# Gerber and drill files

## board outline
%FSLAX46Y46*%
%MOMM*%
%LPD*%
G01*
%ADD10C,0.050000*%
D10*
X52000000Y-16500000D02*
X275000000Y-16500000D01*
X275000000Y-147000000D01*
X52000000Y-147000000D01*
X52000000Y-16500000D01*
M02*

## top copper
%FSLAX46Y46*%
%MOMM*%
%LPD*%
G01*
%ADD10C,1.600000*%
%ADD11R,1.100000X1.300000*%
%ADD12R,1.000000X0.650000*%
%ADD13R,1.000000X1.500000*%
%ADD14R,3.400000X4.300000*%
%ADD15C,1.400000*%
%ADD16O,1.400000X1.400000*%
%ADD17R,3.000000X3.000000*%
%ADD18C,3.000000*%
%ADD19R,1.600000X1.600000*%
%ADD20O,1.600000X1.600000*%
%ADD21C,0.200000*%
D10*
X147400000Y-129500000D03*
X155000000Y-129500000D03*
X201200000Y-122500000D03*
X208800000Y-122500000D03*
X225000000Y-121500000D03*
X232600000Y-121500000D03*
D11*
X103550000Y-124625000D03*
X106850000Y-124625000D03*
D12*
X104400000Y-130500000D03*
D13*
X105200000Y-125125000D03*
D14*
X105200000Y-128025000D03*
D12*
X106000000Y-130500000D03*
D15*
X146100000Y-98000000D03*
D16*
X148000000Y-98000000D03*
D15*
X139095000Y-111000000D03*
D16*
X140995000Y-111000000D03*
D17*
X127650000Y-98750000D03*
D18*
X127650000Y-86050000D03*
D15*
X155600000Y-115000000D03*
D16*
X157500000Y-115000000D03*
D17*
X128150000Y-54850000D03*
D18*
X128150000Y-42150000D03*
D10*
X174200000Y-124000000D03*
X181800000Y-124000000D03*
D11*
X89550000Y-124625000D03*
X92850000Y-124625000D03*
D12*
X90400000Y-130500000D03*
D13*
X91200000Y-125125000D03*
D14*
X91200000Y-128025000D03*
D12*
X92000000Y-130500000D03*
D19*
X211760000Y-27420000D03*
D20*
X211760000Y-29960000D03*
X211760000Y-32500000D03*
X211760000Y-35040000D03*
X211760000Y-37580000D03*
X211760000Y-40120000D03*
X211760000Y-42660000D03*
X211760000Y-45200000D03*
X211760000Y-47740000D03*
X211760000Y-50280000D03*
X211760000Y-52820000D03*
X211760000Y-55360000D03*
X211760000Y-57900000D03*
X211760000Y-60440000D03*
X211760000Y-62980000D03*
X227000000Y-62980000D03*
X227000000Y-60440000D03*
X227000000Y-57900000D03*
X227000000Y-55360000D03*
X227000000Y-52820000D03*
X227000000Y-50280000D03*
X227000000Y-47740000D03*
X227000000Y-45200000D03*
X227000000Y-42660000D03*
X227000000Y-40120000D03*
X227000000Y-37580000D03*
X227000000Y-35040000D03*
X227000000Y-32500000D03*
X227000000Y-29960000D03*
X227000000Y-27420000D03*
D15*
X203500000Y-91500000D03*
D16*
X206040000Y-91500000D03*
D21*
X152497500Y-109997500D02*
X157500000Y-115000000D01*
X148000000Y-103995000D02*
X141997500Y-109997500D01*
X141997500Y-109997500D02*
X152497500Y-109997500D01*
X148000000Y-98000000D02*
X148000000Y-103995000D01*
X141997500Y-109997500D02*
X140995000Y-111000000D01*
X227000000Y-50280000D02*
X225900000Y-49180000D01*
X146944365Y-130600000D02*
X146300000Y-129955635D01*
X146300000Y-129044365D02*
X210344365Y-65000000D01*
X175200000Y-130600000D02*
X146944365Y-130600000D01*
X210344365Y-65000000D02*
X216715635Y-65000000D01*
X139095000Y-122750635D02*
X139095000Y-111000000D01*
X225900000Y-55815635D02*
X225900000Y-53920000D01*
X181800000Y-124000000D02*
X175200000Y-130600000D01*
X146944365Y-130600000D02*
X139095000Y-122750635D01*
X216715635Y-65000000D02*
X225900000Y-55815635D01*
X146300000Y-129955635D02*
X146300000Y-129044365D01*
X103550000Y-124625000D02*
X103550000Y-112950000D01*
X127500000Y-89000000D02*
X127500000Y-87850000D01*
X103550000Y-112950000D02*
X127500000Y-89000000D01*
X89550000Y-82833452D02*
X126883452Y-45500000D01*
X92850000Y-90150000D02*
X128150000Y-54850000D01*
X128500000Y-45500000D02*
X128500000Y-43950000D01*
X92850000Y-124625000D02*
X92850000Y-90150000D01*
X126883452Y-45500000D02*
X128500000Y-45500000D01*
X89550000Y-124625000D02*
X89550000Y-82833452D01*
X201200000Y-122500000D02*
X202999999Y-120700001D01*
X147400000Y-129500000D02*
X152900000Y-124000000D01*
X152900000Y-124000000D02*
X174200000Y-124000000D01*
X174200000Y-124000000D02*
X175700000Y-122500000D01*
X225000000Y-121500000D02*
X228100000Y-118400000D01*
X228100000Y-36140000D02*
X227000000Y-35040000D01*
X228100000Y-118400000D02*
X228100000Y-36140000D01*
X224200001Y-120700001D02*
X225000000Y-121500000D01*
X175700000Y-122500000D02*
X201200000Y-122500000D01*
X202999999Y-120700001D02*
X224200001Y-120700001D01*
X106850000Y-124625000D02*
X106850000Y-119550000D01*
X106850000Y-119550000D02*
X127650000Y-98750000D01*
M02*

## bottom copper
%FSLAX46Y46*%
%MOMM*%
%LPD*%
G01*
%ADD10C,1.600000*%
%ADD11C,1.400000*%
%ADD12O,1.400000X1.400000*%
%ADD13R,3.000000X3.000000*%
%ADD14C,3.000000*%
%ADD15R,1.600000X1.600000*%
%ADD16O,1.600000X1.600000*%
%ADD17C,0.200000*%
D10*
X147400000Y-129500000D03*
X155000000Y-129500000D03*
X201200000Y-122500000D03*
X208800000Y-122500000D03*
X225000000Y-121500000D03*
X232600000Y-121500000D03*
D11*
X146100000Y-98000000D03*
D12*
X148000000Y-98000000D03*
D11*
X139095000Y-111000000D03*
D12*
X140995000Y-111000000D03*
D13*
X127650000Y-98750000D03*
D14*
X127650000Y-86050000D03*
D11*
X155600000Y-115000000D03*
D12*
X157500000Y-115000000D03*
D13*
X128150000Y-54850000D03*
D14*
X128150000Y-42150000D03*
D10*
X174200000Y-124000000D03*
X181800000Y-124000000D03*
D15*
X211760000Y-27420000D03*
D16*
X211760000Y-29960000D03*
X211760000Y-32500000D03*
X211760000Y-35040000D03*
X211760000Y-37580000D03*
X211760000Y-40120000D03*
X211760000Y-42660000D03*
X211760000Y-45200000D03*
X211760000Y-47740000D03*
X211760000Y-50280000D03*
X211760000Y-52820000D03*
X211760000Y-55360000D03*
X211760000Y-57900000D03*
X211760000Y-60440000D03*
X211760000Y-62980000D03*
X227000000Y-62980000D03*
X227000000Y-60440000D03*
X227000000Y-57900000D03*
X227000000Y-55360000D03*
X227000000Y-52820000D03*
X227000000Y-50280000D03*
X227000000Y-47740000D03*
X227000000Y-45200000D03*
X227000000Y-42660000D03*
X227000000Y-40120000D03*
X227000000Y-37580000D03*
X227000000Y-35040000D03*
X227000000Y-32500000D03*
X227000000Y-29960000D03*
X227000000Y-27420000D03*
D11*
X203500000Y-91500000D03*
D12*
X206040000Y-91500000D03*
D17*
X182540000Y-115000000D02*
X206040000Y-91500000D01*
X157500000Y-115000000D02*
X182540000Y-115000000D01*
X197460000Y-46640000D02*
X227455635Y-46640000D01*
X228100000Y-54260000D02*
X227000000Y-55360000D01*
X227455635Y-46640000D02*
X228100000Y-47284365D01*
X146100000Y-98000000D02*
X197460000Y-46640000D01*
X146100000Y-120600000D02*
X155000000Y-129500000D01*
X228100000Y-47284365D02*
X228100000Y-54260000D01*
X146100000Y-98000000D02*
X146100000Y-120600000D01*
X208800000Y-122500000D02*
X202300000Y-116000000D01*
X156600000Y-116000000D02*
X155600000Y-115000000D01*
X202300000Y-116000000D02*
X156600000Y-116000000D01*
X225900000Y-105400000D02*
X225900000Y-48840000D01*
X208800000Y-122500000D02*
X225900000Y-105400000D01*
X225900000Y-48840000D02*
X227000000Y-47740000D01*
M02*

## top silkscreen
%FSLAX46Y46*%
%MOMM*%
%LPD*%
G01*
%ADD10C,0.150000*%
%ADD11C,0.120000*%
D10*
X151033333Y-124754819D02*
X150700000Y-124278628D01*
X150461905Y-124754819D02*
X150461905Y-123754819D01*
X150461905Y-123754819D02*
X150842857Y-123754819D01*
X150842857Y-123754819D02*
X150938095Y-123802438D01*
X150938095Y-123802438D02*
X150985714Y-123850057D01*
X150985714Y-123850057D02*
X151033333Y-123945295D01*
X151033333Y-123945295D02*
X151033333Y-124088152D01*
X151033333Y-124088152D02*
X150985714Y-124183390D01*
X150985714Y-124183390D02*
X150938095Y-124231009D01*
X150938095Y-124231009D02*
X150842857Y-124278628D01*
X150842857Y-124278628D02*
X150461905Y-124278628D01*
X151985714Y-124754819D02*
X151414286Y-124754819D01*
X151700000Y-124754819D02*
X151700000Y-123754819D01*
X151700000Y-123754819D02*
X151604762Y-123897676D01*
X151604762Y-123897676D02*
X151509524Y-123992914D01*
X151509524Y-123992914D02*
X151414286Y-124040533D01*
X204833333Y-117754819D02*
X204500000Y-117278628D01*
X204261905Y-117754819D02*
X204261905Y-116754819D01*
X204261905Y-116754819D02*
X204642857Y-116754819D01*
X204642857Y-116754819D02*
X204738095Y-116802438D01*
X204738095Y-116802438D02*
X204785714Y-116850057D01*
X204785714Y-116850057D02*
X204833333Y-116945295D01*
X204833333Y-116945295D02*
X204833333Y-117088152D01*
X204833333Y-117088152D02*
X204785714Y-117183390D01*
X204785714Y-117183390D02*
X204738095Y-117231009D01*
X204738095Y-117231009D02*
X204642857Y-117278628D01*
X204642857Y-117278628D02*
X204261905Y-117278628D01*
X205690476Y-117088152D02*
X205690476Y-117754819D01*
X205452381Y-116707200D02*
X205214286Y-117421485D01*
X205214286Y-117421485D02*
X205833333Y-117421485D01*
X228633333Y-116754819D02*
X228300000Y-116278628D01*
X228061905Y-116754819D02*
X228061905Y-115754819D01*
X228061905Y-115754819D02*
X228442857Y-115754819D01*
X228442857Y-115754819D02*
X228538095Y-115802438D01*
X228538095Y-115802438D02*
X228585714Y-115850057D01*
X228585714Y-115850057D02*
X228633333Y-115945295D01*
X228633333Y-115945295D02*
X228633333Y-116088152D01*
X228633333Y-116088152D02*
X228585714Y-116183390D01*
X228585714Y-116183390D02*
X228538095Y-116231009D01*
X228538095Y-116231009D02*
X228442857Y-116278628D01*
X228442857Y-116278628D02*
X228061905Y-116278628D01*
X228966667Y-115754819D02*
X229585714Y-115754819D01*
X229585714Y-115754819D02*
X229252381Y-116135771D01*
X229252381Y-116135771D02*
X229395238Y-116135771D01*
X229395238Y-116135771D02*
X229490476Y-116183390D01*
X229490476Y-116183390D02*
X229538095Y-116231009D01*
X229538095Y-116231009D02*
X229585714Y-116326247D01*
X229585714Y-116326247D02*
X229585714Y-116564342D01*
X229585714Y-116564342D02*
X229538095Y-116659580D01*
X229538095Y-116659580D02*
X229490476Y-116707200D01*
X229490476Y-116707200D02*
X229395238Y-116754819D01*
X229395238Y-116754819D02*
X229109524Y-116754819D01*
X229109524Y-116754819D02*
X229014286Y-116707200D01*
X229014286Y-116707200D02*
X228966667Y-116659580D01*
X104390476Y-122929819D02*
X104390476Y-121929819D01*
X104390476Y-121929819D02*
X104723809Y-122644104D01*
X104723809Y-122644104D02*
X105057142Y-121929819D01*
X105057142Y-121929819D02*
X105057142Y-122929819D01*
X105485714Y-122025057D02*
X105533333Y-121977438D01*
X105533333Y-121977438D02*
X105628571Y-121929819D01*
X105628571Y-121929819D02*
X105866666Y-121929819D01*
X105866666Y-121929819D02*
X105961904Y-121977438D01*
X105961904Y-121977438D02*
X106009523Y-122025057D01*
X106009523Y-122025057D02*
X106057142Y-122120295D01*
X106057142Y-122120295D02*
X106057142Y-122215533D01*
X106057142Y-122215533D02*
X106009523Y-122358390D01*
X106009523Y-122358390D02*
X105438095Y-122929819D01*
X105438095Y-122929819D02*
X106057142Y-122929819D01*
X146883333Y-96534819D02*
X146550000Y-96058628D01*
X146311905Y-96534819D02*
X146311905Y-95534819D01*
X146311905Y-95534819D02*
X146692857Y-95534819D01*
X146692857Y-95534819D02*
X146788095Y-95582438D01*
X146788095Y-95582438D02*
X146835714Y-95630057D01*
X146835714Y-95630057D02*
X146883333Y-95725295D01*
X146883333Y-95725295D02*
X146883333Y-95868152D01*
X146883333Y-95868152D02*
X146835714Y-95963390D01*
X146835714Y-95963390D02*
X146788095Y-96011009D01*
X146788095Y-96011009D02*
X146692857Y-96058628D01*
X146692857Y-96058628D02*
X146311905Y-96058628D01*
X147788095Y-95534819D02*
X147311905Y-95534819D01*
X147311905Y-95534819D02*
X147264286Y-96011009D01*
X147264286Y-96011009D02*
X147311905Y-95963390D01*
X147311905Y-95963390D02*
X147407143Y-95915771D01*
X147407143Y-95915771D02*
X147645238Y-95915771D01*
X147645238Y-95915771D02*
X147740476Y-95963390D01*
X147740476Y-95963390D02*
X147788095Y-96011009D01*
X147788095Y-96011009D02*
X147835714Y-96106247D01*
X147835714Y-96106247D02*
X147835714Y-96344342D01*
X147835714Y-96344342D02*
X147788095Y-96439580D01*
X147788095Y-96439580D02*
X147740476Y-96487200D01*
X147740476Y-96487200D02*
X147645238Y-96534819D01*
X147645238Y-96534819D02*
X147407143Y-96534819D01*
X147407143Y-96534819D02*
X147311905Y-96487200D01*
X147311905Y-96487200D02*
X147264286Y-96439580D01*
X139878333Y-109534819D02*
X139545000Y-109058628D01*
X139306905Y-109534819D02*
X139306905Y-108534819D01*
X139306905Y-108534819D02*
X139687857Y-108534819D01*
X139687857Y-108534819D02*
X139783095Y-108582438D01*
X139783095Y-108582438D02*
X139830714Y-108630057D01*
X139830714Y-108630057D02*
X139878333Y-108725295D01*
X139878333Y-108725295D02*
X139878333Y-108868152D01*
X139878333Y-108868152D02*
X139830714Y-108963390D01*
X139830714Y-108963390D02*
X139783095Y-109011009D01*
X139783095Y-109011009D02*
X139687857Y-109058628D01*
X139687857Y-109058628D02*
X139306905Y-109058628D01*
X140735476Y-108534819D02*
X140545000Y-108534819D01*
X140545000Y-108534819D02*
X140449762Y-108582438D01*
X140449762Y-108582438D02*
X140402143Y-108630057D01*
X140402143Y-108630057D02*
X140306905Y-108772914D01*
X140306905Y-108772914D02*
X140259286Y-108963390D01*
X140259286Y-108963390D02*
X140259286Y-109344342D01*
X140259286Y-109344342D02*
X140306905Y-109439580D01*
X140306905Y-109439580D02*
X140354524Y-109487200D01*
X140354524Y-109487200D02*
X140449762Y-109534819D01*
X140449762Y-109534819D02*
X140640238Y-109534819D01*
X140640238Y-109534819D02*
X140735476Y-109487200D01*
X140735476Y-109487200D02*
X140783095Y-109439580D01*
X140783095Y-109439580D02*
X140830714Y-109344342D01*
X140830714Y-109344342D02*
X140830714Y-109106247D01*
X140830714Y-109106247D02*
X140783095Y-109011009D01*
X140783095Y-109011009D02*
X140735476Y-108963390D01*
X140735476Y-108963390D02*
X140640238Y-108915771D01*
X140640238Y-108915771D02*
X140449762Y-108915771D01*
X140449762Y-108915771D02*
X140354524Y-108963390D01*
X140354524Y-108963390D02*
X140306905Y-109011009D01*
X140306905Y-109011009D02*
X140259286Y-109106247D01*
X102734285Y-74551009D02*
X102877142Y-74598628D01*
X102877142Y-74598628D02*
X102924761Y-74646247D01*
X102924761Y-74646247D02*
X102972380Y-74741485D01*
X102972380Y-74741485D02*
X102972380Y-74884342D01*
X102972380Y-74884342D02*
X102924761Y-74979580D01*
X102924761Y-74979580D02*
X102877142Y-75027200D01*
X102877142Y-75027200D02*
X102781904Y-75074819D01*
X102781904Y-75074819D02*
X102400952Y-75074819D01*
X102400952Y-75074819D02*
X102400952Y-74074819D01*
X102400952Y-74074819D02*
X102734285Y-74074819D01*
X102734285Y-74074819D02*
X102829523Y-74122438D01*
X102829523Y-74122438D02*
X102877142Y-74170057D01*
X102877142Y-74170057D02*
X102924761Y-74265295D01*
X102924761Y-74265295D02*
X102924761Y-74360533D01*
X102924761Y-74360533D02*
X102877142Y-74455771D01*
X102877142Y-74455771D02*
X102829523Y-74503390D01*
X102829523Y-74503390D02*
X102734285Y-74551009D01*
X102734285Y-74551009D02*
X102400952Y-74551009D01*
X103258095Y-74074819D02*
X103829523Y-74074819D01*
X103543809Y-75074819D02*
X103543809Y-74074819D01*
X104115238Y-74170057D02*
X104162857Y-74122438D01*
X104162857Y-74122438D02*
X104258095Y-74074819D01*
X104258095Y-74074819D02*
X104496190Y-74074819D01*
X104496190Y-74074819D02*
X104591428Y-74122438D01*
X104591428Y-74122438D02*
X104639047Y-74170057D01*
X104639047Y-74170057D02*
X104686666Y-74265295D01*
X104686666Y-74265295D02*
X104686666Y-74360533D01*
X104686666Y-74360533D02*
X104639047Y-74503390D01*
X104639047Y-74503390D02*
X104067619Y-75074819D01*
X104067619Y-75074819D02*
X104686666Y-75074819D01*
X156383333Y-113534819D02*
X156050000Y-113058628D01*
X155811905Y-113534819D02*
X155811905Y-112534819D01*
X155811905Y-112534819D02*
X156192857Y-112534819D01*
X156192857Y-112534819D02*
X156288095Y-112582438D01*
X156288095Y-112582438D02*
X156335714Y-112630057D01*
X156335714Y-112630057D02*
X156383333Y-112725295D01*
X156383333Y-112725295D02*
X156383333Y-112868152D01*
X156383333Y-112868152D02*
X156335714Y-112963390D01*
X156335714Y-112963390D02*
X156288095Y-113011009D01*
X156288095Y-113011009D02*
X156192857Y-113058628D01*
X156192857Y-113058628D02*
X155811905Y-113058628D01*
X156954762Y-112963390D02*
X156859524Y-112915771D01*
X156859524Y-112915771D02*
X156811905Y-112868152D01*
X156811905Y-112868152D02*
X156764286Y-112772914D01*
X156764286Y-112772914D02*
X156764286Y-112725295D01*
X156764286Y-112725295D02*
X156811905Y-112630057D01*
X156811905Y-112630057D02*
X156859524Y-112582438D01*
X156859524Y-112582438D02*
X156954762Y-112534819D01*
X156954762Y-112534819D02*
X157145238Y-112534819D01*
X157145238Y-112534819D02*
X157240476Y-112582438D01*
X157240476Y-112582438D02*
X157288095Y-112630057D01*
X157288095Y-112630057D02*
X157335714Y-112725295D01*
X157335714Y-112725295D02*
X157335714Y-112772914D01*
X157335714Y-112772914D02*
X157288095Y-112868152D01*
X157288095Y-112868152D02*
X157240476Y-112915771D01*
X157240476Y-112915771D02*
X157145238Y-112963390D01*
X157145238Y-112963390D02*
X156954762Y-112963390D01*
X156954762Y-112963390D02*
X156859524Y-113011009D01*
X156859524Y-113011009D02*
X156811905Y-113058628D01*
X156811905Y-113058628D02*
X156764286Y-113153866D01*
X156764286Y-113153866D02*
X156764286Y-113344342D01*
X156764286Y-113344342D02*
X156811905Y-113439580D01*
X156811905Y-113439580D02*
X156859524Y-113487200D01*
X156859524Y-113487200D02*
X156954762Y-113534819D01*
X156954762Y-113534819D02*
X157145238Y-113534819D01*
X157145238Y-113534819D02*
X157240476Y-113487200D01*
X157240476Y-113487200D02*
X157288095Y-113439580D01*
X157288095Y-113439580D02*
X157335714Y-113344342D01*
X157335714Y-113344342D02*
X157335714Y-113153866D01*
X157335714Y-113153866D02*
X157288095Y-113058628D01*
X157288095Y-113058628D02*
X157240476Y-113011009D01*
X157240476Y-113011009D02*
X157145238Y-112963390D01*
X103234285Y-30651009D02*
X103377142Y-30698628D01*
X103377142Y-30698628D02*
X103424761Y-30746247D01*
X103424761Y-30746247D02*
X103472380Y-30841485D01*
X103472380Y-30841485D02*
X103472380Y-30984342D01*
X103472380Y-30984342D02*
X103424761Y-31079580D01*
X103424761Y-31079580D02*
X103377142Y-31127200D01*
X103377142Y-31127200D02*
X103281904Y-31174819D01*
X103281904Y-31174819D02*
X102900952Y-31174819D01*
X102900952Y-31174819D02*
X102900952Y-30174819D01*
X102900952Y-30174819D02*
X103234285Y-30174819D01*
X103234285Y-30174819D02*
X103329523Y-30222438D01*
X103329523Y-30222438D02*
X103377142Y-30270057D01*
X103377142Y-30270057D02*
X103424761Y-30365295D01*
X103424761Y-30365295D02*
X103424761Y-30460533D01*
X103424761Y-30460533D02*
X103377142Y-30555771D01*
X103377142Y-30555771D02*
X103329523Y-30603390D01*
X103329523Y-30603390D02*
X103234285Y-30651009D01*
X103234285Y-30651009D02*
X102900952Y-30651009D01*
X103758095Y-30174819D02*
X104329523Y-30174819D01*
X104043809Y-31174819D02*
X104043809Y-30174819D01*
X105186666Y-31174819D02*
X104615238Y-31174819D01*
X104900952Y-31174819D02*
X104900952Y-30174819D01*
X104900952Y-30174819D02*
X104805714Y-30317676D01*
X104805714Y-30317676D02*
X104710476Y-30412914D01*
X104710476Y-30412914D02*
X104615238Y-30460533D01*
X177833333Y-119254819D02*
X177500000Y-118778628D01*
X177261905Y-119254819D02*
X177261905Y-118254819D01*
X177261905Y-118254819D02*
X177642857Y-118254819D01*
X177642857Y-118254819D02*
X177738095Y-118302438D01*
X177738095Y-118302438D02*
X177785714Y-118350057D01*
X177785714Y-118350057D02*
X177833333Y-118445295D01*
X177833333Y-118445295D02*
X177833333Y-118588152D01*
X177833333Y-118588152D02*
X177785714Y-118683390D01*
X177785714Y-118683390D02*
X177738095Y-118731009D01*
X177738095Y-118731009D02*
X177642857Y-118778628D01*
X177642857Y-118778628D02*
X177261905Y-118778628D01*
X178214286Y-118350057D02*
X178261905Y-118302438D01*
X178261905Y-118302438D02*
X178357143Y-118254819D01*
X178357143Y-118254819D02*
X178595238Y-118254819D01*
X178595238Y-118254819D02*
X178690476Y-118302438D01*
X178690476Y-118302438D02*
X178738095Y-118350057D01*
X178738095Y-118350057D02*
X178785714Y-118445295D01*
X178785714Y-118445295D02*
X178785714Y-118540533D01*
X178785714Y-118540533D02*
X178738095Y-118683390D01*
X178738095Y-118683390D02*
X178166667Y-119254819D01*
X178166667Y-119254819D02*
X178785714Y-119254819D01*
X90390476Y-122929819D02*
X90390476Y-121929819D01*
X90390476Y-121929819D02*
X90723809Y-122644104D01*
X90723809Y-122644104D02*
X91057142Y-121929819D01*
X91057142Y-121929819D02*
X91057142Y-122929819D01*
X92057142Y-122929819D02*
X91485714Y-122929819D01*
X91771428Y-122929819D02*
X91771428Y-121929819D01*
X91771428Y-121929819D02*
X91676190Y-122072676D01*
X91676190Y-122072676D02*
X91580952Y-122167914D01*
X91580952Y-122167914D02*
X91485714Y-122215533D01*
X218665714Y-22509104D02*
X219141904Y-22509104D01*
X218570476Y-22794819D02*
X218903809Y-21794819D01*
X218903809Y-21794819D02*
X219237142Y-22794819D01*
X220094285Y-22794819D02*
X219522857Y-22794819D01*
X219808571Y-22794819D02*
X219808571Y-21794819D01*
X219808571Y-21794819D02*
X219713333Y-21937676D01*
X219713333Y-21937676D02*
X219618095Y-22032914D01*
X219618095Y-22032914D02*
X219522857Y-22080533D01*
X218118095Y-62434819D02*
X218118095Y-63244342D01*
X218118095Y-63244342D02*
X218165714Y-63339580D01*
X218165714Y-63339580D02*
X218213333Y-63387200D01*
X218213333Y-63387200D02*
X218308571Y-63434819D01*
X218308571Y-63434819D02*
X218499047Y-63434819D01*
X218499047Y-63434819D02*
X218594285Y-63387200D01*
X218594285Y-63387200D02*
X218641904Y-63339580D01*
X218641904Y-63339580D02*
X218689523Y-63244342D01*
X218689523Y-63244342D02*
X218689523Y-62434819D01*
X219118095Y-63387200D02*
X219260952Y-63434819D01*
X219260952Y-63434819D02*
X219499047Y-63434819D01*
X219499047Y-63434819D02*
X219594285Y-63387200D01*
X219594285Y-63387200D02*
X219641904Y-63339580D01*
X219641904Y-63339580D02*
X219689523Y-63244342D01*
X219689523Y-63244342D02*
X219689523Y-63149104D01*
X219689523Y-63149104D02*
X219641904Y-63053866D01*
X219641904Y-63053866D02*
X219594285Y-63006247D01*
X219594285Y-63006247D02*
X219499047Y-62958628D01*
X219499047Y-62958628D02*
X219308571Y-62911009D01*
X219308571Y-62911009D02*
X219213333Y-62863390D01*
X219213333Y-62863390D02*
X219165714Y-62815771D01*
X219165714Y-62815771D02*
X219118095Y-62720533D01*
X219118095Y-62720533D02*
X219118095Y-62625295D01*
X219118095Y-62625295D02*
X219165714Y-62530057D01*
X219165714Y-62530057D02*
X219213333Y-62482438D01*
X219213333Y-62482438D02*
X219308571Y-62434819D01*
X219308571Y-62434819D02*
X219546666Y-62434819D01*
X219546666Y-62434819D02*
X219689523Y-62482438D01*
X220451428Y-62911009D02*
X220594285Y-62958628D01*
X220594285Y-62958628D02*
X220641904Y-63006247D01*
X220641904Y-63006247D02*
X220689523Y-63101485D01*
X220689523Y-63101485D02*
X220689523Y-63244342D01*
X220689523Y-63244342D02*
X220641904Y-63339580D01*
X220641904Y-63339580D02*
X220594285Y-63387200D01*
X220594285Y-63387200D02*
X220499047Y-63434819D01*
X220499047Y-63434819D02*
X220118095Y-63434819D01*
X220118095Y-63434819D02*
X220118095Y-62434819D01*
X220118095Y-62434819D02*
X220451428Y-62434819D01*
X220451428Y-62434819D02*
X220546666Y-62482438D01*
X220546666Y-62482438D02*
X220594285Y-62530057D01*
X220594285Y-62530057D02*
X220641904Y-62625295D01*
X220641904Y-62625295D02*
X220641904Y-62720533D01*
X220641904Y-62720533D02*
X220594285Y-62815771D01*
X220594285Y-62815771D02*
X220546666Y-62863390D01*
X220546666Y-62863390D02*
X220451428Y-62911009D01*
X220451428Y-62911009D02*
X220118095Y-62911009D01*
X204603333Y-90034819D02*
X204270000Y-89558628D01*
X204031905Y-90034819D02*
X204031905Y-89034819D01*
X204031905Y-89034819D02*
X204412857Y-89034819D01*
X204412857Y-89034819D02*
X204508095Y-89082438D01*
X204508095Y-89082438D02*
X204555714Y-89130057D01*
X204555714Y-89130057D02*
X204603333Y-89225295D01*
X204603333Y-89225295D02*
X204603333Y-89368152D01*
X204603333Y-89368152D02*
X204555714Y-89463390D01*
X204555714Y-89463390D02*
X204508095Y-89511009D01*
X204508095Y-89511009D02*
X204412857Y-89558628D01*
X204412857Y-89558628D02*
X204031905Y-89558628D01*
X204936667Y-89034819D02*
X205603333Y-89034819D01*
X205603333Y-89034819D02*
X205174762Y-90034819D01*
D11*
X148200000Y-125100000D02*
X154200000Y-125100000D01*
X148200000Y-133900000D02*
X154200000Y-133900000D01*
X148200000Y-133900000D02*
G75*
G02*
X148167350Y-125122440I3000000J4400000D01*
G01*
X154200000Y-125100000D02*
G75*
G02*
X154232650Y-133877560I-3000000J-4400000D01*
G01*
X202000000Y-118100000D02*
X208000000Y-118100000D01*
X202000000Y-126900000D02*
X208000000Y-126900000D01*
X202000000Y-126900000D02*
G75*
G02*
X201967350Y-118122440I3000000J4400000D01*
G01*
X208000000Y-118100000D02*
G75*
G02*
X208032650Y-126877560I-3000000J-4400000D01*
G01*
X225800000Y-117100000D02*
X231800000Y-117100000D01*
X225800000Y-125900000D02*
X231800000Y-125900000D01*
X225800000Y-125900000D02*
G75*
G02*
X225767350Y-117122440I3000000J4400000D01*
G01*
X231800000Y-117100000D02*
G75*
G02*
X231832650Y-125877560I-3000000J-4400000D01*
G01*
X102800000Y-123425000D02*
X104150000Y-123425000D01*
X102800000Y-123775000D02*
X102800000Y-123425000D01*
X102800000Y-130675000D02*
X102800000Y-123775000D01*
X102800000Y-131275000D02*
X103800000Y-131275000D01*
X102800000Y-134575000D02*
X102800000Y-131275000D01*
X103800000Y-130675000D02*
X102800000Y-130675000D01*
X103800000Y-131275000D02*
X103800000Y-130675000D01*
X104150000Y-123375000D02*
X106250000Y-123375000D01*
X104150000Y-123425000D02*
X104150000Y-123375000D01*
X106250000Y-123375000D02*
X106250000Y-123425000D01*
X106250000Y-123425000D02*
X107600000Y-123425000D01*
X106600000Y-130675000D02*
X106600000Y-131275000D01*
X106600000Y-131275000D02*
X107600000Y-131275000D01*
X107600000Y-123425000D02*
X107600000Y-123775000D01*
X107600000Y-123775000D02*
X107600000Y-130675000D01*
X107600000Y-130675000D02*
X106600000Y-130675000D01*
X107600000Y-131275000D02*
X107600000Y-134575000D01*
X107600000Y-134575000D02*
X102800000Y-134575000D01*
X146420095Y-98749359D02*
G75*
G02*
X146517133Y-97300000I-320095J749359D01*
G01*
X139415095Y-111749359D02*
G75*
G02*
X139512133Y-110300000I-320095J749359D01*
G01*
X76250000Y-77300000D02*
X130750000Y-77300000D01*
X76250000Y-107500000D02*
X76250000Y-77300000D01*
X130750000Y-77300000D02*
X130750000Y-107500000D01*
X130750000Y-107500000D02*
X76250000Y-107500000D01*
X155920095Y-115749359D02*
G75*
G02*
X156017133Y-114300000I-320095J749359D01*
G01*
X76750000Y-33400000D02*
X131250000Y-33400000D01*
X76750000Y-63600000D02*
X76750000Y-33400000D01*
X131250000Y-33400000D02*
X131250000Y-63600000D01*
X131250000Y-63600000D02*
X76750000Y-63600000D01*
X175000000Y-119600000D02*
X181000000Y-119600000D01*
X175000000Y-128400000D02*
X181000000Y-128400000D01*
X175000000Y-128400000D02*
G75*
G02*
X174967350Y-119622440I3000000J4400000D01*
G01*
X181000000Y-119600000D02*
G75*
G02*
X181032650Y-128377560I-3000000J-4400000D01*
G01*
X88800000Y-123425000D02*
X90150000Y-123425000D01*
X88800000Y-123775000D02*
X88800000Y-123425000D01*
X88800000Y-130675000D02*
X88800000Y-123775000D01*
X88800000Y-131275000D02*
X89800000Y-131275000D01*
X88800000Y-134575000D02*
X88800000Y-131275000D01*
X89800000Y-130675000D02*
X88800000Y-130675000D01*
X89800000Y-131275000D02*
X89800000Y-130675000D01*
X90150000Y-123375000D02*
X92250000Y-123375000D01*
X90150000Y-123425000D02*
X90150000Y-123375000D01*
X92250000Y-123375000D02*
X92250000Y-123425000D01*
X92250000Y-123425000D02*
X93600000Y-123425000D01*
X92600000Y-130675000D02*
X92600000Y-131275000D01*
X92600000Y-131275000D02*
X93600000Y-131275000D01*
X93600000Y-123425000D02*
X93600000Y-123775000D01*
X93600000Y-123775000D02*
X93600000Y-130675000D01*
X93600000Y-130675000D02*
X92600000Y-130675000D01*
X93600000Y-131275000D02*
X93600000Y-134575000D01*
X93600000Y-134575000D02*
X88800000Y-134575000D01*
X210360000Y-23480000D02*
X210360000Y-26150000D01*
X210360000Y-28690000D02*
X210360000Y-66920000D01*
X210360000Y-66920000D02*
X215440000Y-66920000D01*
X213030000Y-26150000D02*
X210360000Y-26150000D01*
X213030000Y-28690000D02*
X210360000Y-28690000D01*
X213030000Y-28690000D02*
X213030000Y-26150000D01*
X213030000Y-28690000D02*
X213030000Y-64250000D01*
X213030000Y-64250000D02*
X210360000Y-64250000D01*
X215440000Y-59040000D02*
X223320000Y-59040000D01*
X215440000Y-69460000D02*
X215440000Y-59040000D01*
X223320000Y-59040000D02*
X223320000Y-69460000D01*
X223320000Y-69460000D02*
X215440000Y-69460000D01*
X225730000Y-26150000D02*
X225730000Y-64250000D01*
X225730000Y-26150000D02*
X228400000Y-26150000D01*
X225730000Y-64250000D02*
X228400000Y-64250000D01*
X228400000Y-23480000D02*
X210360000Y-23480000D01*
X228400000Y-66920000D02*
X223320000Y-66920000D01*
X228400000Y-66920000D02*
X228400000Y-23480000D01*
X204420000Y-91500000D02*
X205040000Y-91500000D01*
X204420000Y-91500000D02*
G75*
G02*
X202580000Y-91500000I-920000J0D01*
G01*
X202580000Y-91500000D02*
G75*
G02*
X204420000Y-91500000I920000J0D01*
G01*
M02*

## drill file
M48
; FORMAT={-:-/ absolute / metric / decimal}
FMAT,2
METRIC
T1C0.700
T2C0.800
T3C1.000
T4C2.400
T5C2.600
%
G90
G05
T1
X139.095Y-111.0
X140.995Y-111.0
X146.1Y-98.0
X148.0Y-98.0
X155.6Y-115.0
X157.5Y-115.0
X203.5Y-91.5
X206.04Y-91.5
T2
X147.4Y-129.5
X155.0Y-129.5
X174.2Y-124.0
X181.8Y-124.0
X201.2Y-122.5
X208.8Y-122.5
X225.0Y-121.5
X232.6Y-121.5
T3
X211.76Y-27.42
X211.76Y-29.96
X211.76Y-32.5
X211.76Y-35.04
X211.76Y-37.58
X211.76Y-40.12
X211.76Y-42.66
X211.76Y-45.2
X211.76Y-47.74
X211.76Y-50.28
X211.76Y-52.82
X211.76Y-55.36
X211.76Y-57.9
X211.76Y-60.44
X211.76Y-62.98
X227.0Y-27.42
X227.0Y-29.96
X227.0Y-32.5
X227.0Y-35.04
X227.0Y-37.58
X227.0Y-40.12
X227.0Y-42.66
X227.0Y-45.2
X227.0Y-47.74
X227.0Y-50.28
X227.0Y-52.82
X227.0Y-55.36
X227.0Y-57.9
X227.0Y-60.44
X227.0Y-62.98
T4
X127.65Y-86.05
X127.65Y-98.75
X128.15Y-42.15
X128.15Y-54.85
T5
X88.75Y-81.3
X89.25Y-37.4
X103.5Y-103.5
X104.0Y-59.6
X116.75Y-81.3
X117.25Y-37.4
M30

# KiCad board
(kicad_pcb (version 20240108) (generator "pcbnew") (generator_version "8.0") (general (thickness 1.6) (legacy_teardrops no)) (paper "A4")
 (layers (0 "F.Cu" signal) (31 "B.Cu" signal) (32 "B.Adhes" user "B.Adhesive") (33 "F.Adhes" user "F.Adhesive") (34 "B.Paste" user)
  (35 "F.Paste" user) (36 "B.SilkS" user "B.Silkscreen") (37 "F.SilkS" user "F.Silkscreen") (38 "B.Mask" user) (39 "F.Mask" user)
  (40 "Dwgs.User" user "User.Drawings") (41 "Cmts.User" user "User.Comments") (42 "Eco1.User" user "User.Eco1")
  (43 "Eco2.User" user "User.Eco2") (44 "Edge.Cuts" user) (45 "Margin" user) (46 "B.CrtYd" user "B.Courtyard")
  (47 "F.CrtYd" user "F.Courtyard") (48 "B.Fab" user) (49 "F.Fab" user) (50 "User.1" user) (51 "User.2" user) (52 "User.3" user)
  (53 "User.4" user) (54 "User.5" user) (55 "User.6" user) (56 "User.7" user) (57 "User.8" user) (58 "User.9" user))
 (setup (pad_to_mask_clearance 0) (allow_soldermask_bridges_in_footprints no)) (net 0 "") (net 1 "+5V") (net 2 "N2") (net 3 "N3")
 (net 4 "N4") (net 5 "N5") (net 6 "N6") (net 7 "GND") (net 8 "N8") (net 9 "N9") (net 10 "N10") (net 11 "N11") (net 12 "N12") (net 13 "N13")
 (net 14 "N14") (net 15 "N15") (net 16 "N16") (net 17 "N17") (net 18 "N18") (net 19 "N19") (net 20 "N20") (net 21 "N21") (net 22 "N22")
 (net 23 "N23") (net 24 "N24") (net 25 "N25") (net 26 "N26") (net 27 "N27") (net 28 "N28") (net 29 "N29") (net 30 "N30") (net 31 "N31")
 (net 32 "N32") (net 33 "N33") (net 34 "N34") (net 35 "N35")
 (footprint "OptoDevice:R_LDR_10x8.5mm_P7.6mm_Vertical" (layer "F.Cu") (at 147.4 129.5)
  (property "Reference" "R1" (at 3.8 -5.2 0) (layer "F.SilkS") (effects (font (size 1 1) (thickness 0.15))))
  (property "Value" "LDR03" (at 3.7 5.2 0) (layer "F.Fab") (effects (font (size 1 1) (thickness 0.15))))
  (fp_line (start 0.8 -4.4) (end 6.8 -4.4) (stroke (width 0.12) (type solid)) (layer "F.SilkS"))
  (fp_line (start 0.8 4.4) (end 6.8 4.4) (stroke (width 0.12) (type solid)) (layer "F.SilkS"))
  (fp_arc (start 0.8 4.4) (mid -1.525374 0.019809) (end 0.76735 -4.37756) (stroke (width 0.12) (type solid)) (layer "F.SilkS"))
  (fp_arc (start 6.8 -4.4) (mid 9.125374 -0.019809) (end 6.83265 4.37756) (stroke (width 0.12) (type solid)) (layer "F.SilkS"))
  (pad "1" thru_hole circle (at 0 0) (size 1.6 1.6) (drill 0.8) (layers "*.Cu" "*.Mask") (remove_unused_layers no) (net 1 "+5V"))
  (pad "2" thru_hole circle (at 7.6 0) (size 1.6 1.6) (drill 0.8) (layers "*.Cu" "*.Mask") (remove_unused_layers no) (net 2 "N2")))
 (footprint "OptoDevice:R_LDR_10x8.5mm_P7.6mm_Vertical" (layer "F.Cu") (at 201.2 122.5)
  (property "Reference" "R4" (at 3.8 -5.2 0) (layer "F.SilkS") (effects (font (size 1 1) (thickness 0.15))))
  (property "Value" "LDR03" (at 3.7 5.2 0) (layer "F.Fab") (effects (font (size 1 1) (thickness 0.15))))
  (fp_line (start 0.8 -4.4) (end 6.8 -4.4) (stroke (width 0.12) (type solid)) (layer "F.SilkS"))
  (fp_line (start 0.8 4.4) (end 6.8 4.4) (stroke (width 0.12) (type solid)) (layer "F.SilkS"))
  (fp_arc (start 0.8 4.4) (mid -1.525374 0.019809) (end 0.76735 -4.37756) (stroke (width 0.12) (type solid)) (layer "F.SilkS"))
  (fp_arc (start 6.8 -4.4) (mid 9.125374 -0.019809) (end 6.83265 4.37756) (stroke (width 0.12) (type solid)) (layer "F.SilkS"))
  (pad "1" thru_hole circle (at 0 0) (size 1.6 1.6) (drill 0.8) (layers "*.Cu" "*.Mask") (remove_unused_layers no) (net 1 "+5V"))
  (pad "2" thru_hole circle (at 7.6 0) (size 1.6 1.6) (drill 0.8) (layers "*.Cu" "*.Mask") (remove_unused_layers no) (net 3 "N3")))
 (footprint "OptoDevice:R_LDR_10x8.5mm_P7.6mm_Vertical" (layer "F.Cu") (at 225 121.5)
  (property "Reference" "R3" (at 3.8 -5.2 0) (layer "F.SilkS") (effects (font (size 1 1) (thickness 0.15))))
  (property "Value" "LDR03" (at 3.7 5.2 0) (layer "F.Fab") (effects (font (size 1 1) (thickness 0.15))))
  (fp_line (start 0.8 -4.4) (end 6.8 -4.4) (stroke (width 0.12) (type solid)) (layer "F.SilkS"))
  (fp_line (start 0.8 4.4) (end 6.8 4.4) (stroke (width 0.12) (type solid)) (layer "F.SilkS"))
  (fp_arc (start 0.8 4.4) (mid -1.525374 0.019809) (end 0.76735 -4.37756) (stroke (width 0.12) (type solid)) (layer "F.SilkS"))
  (fp_arc (start 6.8 -4.4) (mid 9.125374 -0.019809) (end 6.83265 4.37756) (stroke (width 0.12) (type solid)) (layer "F.SilkS"))
  (pad "1" thru_hole circle (at 0 0) (size 1.6 1.6) (drill 0.8) (layers "*.Cu" "*.Mask") (remove_unused_layers no) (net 1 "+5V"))
  (pad "2" thru_hole circle (at 7.6 0) (size 1.6 1.6) (drill 0.8) (layers "*.Cu" "*.Mask") (remove_unused_layers no) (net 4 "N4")))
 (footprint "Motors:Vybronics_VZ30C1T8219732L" (layer "F.Cu") (at 105.2 128.975)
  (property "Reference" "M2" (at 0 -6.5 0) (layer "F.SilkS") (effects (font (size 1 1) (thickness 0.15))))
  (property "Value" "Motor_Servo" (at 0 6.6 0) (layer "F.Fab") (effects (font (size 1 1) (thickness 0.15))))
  (fp_line (start -2.4 -5.55) (end -1.05 -5.55) (stroke (width 0.12) (type solid)) (layer "F.SilkS"))
  (fp_line (start -2.4 -5.2) (end -2.4 -5.55) (stroke (width 0.12) (type solid)) (layer "F.SilkS"))
  (fp_line (start -2.4 1.7) (end -2.4 -5.2) (stroke (width 0.12) (type solid)) (layer "F.SilkS"))
  (fp_line (start -2.4 2.3) (end -1.4 2.3) (stroke (width 0.12) (type solid)) (layer "F.SilkS"))
  (fp_line (start -2.4 5.6) (end -2.4 2.3) (stroke (width 0.12) (type solid)) (layer "F.SilkS"))
  (fp_line (start -1.4 1.7) (end -2.4 1.7) (stroke (width 0.12) (type solid)) (layer "F.SilkS"))
  (fp_line (start -1.4 2.3) (end -1.4 1.7) (stroke (width 0.12) (type solid)) (layer "F.SilkS"))
  (fp_line (start -1.05 -5.6) (end 1.05 -5.6) (stroke (width 0.12) (type solid)) (layer "F.SilkS"))
  (fp_line (start -1.05 -5.55) (end -1.05 -5.6) (stroke (width 0.12) (type solid)) (layer "F.SilkS"))
  (fp_line (start 1.05 -5.6) (end 1.05 -5.55) (stroke (width 0.12) (type solid)) (layer "F.SilkS"))
  (fp_line (start 1.05 -5.55) (end 2.4 -5.55) (stroke (width 0.12) (type solid)) (layer "F.SilkS"))
  (fp_line (start 1.4 1.7) (end 1.4 2.3) (stroke (width 0.12) (type solid)) (layer "F.SilkS"))
  (fp_line (start 1.4 2.3) (end 2.4 2.3) (stroke (width 0.12) (type solid)) (layer "F.SilkS"))
  (fp_line (start 2.4 -5.55) (end 2.4 -5.2) (stroke (width 0.12) (type solid)) (layer "F.SilkS"))
  (fp_line (start 2.4 -5.2) (end 2.4 1.7) (stroke (width 0.12) (type solid)) (layer "F.SilkS"))
  (fp_line (start 2.4 1.7) (end 1.4 1.7) (stroke (width 0.12) (type solid)) (layer "F.SilkS"))
  (fp_line (start 2.4 2.3) (end 2.4 5.6) (stroke (width 0.12) (type solid)) (layer "F.SilkS"))
  (fp_line (start 2.4 5.6) (end -2.4 5.6) (stroke (width 0.12) (type solid)) (layer "F.SilkS"))
  (pad "" smd rect (at -0.85 -2.315 270) (size 1.07 1.4) (layers "F.Paste"))
  (pad "" smd rect (at -0.85 -0.905 270) (size 1.07 1.4) (layers "F.Paste"))
  (pad "" smd rect (at -0.85 0.505 270) (size 1.07 1.4) (layers "F.Paste"))
  (pad "" smd rect (at 0.85 -2.315 270) (size 1.07 1.4) (layers "F.Paste"))
  (pad "" smd rect (at 0.85 -0.905 270) (size 1.07 1.4) (layers "F.Paste"))
  (pad "" smd rect (at 0.85 0.505 270) (size 1.07 1.4) (layers "F.Paste"))
  (pad "1" smd rect (at -1.65 -4.35 270) (size 1.3 1.1) (layers "F.Cu" "F.Paste" "F.Mask") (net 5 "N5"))
  (pad "2" smd rect (at 1.65 -4.35 270) (size 1.3 1.1) (layers "F.Cu" "F.Paste" "F.Mask") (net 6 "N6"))
  (pad "SH" smd rect (at -0.8 1.525) (size 1 0.65) (layers "F.Cu" "F.Paste" "F.Mask"))
  (pad "SH" smd rect (at 0 -3.85 270) (size 1.5 1) (layers "F.Cu" "F.Paste" "F.Mask"))
  (pad "SH" smd rect (at 0 -0.95 270) (size 4.3 3.4) (layers "F.Cu" "F.Mask"))
  (pad "SH" smd rect (at 0.8 1.525) (size 1 0.65) (layers "F.Cu" "F.Paste" "F.Mask")))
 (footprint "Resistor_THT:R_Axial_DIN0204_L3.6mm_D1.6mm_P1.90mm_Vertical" (layer "F.Cu") (at 146.1 98)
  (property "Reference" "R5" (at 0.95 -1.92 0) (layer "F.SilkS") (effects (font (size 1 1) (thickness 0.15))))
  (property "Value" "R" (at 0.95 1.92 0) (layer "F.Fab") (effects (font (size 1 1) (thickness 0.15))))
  (fp_arc (start 0.320095 0.749359) (mid -0.813042 -0.054435) (end 0.417133 -0.7) (stroke (width 0.12) (type solid)) (layer "F.SilkS"))
  (pad "1" thru_hole circle (at 0 0) (size 1.4 1.4) (drill 0.7) (layers "*.Cu" "*.Mask") (remove_unused_layers no) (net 2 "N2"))
  (pad "2" thru_hole oval (at 1.9 0) (size 1.4 1.4) (drill 0.7) (layers "*.Cu" "*.Mask") (remove_unused_layers no) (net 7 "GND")))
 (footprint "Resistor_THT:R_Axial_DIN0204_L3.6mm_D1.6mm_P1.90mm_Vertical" (layer "F.Cu") (at 139.095 111)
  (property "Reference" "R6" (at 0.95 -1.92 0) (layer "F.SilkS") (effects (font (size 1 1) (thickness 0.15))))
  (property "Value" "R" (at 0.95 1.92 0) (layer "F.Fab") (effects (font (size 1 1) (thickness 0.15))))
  (fp_arc (start 0.320095 0.749359) (mid -0.813042 -0.054435) (end 0.417133 -0.7) (stroke (width 0.12) (type solid)) (layer "F.SilkS"))
  (pad "1" thru_hole circle (at 0 0) (size 1.4 1.4) (drill 0.7) (layers "*.Cu" "*.Mask") (remove_unused_layers no) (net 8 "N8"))
  (pad "2" thru_hole oval (at 1.9 0) (size 1.4 1.4) (drill 0.7) (layers "*.Cu" "*.Mask") (remove_unused_layers no) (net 7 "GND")))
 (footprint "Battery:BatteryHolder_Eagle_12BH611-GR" (layer "F.Cu") (at 127.65 98.75)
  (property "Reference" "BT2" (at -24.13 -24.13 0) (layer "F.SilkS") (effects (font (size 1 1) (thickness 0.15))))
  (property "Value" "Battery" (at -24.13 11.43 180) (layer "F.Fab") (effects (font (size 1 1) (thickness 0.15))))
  (fp_line (start -51.4 -21.45) (end 3.1 -21.45) (stroke (width 0.12) (type solid)) (layer "F.SilkS"))
  (fp_line (start -51.4 8.75) (end -51.4 -21.45) (stroke (width 0.12) (type solid)) (layer "F.SilkS"))
  (fp_line (start 3.1 -21.45) (end 3.1 8.75) (stroke (width 0.12) (type solid)) (layer "F.SilkS"))
  (fp_line (start 3.1 8.75) (end -51.4 8.75) (stroke (width 0.12) (type solid)) (layer "F.SilkS"))
  (pad "" np_thru_hole circle (at -38.9 -17.45) (size 2.6 2.6) (drill 2.6) (layers "*.Cu" "*.Mask"))
  (pad "" np_thru_hole circle (at -24.15 4.75) (size 2.6 2.6) (drill 2.6) (layers "*.Cu" "*.Mask"))
  (pad "" np_thru_hole circle (at -10.9 -17.45) (size 2.6 2.6) (drill 2.6) (layers "*.Cu" "*.Mask"))
  (pad "1" thru_hole rect (at 0 0) (size 3 3) (drill 2.4) (layers "*.Cu" "*.Mask") (remove_unused_layers no) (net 6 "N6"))
  (pad "2" thru_hole circle (at 0 -12.7) (size 3 3) (drill 2.4) (layers "*.Cu" "*.Mask") (remove_unused_layers no) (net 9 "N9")))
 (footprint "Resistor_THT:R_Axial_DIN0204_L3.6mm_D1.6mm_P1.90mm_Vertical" (layer "F.Cu") (at 155.6 115)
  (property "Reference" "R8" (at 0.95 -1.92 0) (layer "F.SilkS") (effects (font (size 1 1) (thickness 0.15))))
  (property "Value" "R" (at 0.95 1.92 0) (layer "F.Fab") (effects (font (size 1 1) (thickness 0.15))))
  (fp_arc (start 0.320095 0.749359) (mid -0.813042 -0.054435) (end 0.417133 -0.7) (stroke (width 0.12) (type solid)) (layer "F.SilkS"))
  (pad "1" thru_hole circle (at 0 0) (size 1.4 1.4) (drill 0.7) (layers "*.Cu" "*.Mask") (remove_unused_layers no) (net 3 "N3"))
  (pad "2" thru_hole oval (at 1.9 0) (size 1.4 1.4) (drill 0.7) (layers "*.Cu" "*.Mask") (remove_unused_layers no) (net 7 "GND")))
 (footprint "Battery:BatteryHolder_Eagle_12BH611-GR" (layer "F.Cu") (at 128.15 54.85)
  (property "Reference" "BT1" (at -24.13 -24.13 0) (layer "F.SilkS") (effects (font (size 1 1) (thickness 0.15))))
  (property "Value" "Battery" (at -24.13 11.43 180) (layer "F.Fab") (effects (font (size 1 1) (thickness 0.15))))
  (fp_line (start -51.4 -21.45) (end 3.1 -21.45) (stroke (width 0.12) (type solid)) (layer "F.SilkS"))
  (fp_line (start -51.4 8.75) (end -51.4 -21.45) (stroke (width 0.12) (type solid)) (layer "F.SilkS"))
  (fp_line (start 3.1 -21.45) (end 3.1 8.75) (stroke (width 0.12) (type solid)) (layer "F.SilkS"))
  (fp_line (start 3.1 8.75) (end -51.4 8.75) (stroke (width 0.12) (type solid)) (layer "F.SilkS"))
  (pad "" np_thru_hole circle (at -38.9 -17.45) (size 2.6 2.6) (drill 2.6) (layers "*.Cu" "*.Mask"))
  (pad "" np_thru_hole circle (at -24.15 4.75) (size 2.6 2.6) (drill 2.6) (layers "*.Cu" "*.Mask"))
  (pad "" np_thru_hole circle (at -10.9 -17.45) (size 2.6 2.6) (drill 2.6) (layers "*.Cu" "*.Mask"))
  (pad "1" thru_hole rect (at 0 0) (size 3 3) (drill 2.4) (layers "*.Cu" "*.Mask") (remove_unused_layers no) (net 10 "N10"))
  (pad "2" thru_hole circle (at 0 -12.7) (size 3 3) (drill 2.4) (layers "*.Cu" "*.Mask") (remove_unused_layers no) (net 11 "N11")))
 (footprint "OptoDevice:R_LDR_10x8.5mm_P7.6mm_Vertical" (layer "F.Cu") (at 174.2 124)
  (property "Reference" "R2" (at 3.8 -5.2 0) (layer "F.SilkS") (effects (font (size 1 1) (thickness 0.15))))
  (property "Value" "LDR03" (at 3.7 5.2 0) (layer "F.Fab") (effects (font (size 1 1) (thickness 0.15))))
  (fp_line (start 0.8 -4.4) (end 6.8 -4.4) (stroke (width 0.12) (type solid)) (layer "F.SilkS"))
  (fp_line (start 0.8 4.4) (end 6.8 4.4) (stroke (width 0.12) (type solid)) (layer "F.SilkS"))
  (fp_arc (start 0.8 4.4) (mid -1.525374 0.019809) (end 0.76735 -4.37756) (stroke (width 0.12) (type solid)) (layer "F.SilkS"))
  (fp_arc (start 6.8 -4.4) (mid 9.125374 -0.019809) (end 6.83265 4.37756) (stroke (width 0.12) (type solid)) (layer "F.SilkS"))
  (pad "1" thru_hole circle (at 0 0) (size 1.6 1.6) (drill 0.8) (layers "*.Cu" "*.Mask") (remove_unused_layers no) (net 1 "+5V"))
  (pad "2" thru_hole circle (at 7.6 0) (size 1.6 1.6) (drill 0.8) (layers "*.Cu" "*.Mask") (remove_unused_layers no) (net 8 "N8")))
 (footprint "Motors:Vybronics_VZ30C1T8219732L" (layer "F.Cu") (at 91.2 128.975)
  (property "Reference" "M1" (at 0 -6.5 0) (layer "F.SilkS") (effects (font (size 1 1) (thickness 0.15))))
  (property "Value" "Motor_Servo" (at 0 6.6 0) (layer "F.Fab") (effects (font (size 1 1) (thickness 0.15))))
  (fp_line (start -2.4 -5.55) (end -1.05 -5.55) (stroke (width 0.12) (type solid)) (layer "F.SilkS"))
  (fp_line (start -2.4 -5.2) (end -2.4 -5.55) (stroke (width 0.12) (type solid)) (layer "F.SilkS"))
  (fp_line (start -2.4 1.7) (end -2.4 -5.2) (stroke (width 0.12) (type solid)) (layer "F.SilkS"))
  (fp_line (start -2.4 2.3) (end -1.4 2.3) (stroke (width 0.12) (type solid)) (layer "F.SilkS"))
  (fp_line (start -2.4 5.6) (end -2.4 2.3) (stroke (width 0.12) (type solid)) (layer "F.SilkS"))
  (fp_line (start -1.4 1.7) (end -2.4 1.7) (stroke (width 0.12) (type solid)) (layer "F.SilkS"))
  (fp_line (start -1.4 2.3) (end -1.4 1.7) (stroke (width 0.12) (type solid)) (layer "F.SilkS"))
  (fp_line (start -1.05 -5.6) (end 1.05 -5.6) (stroke (width 0.12) (type solid)) (layer "F.SilkS"))
  (fp_line (start -1.05 -5.55) (end -1.05 -5.6) (stroke (width 0.12) (type solid)) (layer "F.SilkS"))
  (fp_line (start 1.05 -5.6) (end 1.05 -5.55) (stroke (width 0.12) (type solid)) (layer "F.SilkS"))
  (fp_line (start 1.05 -5.55) (end 2.4 -5.55) (stroke (width 0.12) (type solid)) (layer "F.SilkS"))
  (fp_line (start 1.4 1.7) (end 1.4 2.3) (stroke (width 0.12) (type solid)) (layer "F.SilkS"))
  (fp_line (start 1.4 2.3) (end 2.4 2.3) (stroke (width 0.12) (type solid)) (layer "F.SilkS"))
  (fp_line (start 2.4 -5.55) (end 2.4 -5.2) (stroke (width 0.12) (type solid)) (layer "F.SilkS"))
  (fp_line (start 2.4 -5.2) (end 2.4 1.7) (stroke (width 0.12) (type solid)) (layer "F.SilkS"))
  (fp_line (start 2.4 1.7) (end 1.4 1.7) (stroke (width 0.12) (type solid)) (layer "F.SilkS"))
  (fp_line (start 2.4 2.3) (end 2.4 5.6) (stroke (width 0.12) (type solid)) (layer "F.SilkS"))
  (fp_line (start 2.4 5.6) (end -2.4 5.6) (stroke (width 0.12) (type solid)) (layer "F.SilkS"))
  (pad "" smd rect (at -0.85 -2.315 270) (size 1.07 1.4) (layers "F.Paste"))
  (pad "" smd rect (at -0.85 -0.905 270) (size 1.07 1.4) (layers "F.Paste"))
  (pad "" smd rect (at -0.85 0.505 270) (size 1.07 1.4) (layers "F.Paste"))
  (pad "" smd rect (at 0.85 -2.315 270) (size 1.07 1.4) (layers "F.Paste"))
  (pad "" smd rect (at 0.85 -0.905 270) (size 1.07 1.4) (layers "F.Paste"))
  (pad "" smd rect (at 0.85 0.505 270) (size 1.07 1.4) (layers "F.Paste"))
  (pad "1" smd rect (at -1.65 -4.35 270) (size 1.3 1.1) (layers "F.Cu" "F.Paste" "F.Mask") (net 10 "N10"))
  (pad "2" smd rect (at 1.65 -4.35 270) (size 1.3 1.1) (layers "F.Cu" "F.Paste" "F.Mask") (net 10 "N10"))
  (pad "SH" smd rect (at -0.8 1.525) (size 1 0.65) (layers "F.Cu" "F.Paste" "F.Mask"))
  (pad "SH" smd rect (at 0 -3.85 270) (size 1.5 1) (layers "F.Cu" "F.Paste" "F.Mask"))
  (pad "SH" smd rect (at 0 -0.95 270) (size 4.3 3.4) (layers "F.Cu" "F.Mask"))
  (pad "SH" smd rect (at 0.8 1.525) (size 1 0.65) (layers "F.Cu" "F.Paste" "F.Mask")))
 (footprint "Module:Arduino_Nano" (layer "F.Cu") (at 211.76 27.42)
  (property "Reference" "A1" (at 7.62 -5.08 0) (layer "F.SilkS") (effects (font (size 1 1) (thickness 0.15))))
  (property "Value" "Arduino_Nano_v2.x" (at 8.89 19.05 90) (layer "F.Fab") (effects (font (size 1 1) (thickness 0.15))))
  (fp_line (start -1.4 -3.94) (end -1.4 -1.27) (stroke (width 0.12) (type solid)) (layer "F.SilkS"))
  (fp_line (start -1.4 1.27) (end -1.4 39.5) (stroke (width 0.12) (type solid)) (layer "F.SilkS"))
  (fp_line (start -1.4 39.5) (end 3.68 39.5) (stroke (width 0.12) (type solid)) (layer "F.SilkS"))
  (fp_line (start 1.27 -1.27) (end -1.4 -1.27) (stroke (width 0.12) (type solid)) (layer "F.SilkS"))
  (fp_line (start 1.27 1.27) (end -1.4 1.27) (stroke (width 0.12) (type solid)) (layer "F.SilkS"))
  (fp_line (start 1.27 1.27) (end 1.27 -1.27) (stroke (width 0.12) (type solid)) (layer "F.SilkS"))
  (fp_line (start 1.27 1.27) (end 1.27 36.83) (stroke (width 0.12) (type solid)) (layer "F.SilkS"))
  (fp_line (start 1.27 36.83) (end -1.4 36.83) (stroke (width 0.12) (type solid)) (layer "F.SilkS"))
  (fp_line (start 3.68 31.62) (end 11.56 31.62) (stroke (width 0.12) (type solid)) (layer "F.SilkS"))
  (fp_line (start 3.68 42.04) (end 3.68 31.62) (stroke (width 0.12) (type solid)) (layer "F.SilkS"))
  (fp_line (start 11.56 31.62) (end 11.56 42.04) (stroke (width 0.12) (type solid)) (layer "F.SilkS"))
  (fp_line (start 11.56 42.04) (end 3.68 42.04) (stroke (width 0.12) (type solid)) (layer "F.SilkS"))
  (fp_line (start 13.97 -1.27) (end 13.97 36.83) (stroke (width 0.12) (type solid)) (layer "F.SilkS"))
  (fp_line (start 13.97 -1.27) (end 16.64 -1.27) (stroke (width 0.12) (type solid)) (layer "F.SilkS"))
  (fp_line (start 13.97 36.83) (end 16.64 36.83) (stroke (width 0.12) (type solid)) (layer "F.SilkS"))
  (fp_line (start 16.64 -3.94) (end -1.4 -3.94) (stroke (width 0.12) (type solid)) (layer "F.SilkS"))
  (fp_line (start 16.64 39.5) (end 11.56 39.5) (stroke (width 0.12) (type solid)) (layer "F.SilkS"))
  (fp_line (start 16.64 39.5) (end 16.64 -3.94) (stroke (width 0.12) (type solid)) (layer "F.SilkS"))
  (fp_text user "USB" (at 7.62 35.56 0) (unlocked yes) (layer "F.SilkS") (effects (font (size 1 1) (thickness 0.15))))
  (pad "1" thru_hole rect (at 0 0) (size 1.6 1.6) (drill 1) (layers "*.Cu" "*.Mask") (remove_unused_layers no) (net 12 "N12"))
  (pad "2" thru_hole oval (at 0 2.54) (size 1.6 1.6) (drill 1) (layers "*.Cu" "*.Mask") (remove_unused_layers no) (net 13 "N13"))
  (pad "3" thru_hole oval (at 0 5.08) (size 1.6 1.6) (drill 1) (layers "*.Cu" "*.Mask") (remove_unused_layers no) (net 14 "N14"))
  (pad "4" thru_hole oval (at 0 7.62) (size 1.6 1.6) (drill 1) (layers "*.Cu" "*.Mask") (remove_unused_layers no) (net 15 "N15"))
  (pad "5" thru_hole oval (at 0 10.16) (size 1.6 1.6) (drill 1) (layers "*.Cu" "*.Mask") (remove_unused_layers no) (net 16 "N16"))
  (pad "6" thru_hole oval (at 0 12.7) (size 1.6 1.6) (drill 1) (layers "*.Cu" "*.Mask") (remove_unused_layers no) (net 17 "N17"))
  (pad "7" thru_hole oval (at 0 15.24) (size 1.6 1.6) (drill 1) (layers "*.Cu" "*.Mask") (remove_unused_layers no) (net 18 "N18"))
  (pad "8" thru_hole oval (at 0 17.78) (size 1.6 1.6) (drill 1) (layers "*.Cu" "*.Mask") (remove_unused_layers no) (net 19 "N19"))
  (pad "9" thru_hole oval (at 0 20.32) (size 1.6 1.6) (drill 1) (layers "*.Cu" "*.Mask") (remove_unused_layers no) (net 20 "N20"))
  (pad "10" thru_hole oval (at 0 22.86) (size 1.6 1.6) (drill 1) (layers "*.Cu" "*.Mask") (remove_unused_layers no) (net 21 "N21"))
  (pad "11" thru_hole oval (at 0 25.4) (size 1.6 1.6) (drill 1) (layers "*.Cu" "*.Mask") (remove_unused_layers no) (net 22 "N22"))
  (pad "12" thru_hole oval (at 0 27.94) (size 1.6 1.6) (drill 1) (layers "*.Cu" "*.Mask") (remove_unused_layers no) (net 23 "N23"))
  (pad "13" thru_hole oval (at 0 30.48) (size 1.6 1.6) (drill 1) (layers "*.Cu" "*.Mask") (remove_unused_layers no) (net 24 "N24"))
  (pad "14" thru_hole oval (at 0 33.02) (size 1.6 1.6) (drill 1) (layers "*.Cu" "*.Mask") (remove_unused_layers no) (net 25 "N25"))
  (pad "15" thru_hole oval (at 0 35.56) (size 1.6 1.6) (drill 1) (layers "*.Cu" "*.Mask") (remove_unused_layers no) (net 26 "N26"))
  (pad "16" thru_hole oval (at 15.24 35.56) (size 1.6 1.6) (drill 1) (layers "*.Cu" "*.Mask") (remove_unused_layers no) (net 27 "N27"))
  (pad "17" thru_hole oval (at 15.24 33.02) (size 1.6 1.6) (drill 1) (layers "*.Cu" "*.Mask") (remove_unused_layers no) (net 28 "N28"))
  (pad "18" thru_hole oval (at 15.24 30.48) (size 1.6 1.6) (drill 1) (layers "*.Cu" "*.Mask") (remove_unused_layers no) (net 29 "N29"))
  (pad "19" thru_hole oval (at 15.24 27.94) (size 1.6 1.6) (drill 1) (layers "*.Cu" "*.Mask") (remove_unused_layers no) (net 2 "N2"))
  (pad "20" thru_hole oval (at 15.24 25.4) (size 1.6 1.6) (drill 1) (layers "*.Cu" "*.Mask") (remove_unused_layers no) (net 8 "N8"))
  (pad "21" thru_hole oval (at 15.24 22.86) (size 1.6 1.6) (drill 1) (layers "*.Cu" "*.Mask") (remove_unused_layers no) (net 4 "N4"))
  (pad "22" thru_hole oval (at 15.24 20.32) (size 1.6 1.6) (drill 1) (layers "*.Cu" "*.Mask") (remove_unused_layers no) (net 3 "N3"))
  (pad "23" thru_hole oval (at 15.24 17.78) (size 1.6 1.6) (drill 1) (layers "*.Cu" "*.Mask") (remove_unused_layers no) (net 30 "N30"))
  (pad "24" thru_hole oval (at 15.24 15.24) (size 1.6 1.6) (drill 1) (layers "*.Cu" "*.Mask") (remove_unused_layers no) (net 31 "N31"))
  (pad "25" thru_hole oval (at 15.24 12.7) (size 1.6 1.6) (drill 1) (layers "*.Cu" "*.Mask") (remove_unused_layers no) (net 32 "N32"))
  (pad "26" thru_hole oval (at 15.24 10.16) (size 1.6 1.6) (drill 1) (layers "*.Cu" "*.Mask") (remove_unused_layers no) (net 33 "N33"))
  (pad "27" thru_hole oval (at 15.24 7.62) (size 1.6 1.6) (drill 1) (layers "*.Cu" "*.Mask") (remove_unused_layers no) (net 1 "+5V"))
  (pad "28" thru_hole oval (at 15.24 5.08) (size 1.6 1.6) (drill 1) (layers "*.Cu" "*.Mask") (remove_unused_layers no) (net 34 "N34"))
  (pad "29" thru_hole oval (at 15.24 2.54) (size 1.6 1.6) (drill 1) (layers "*.Cu" "*.Mask") (remove_unused_layers no) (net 7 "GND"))
  (pad "30" thru_hole oval (at 15.24 0) (size 1.6 1.6) (drill 1) (layers "*.Cu" "*.Mask") (remove_unused_layers no) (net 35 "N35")))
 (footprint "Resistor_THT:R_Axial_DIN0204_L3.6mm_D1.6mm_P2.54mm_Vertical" (layer "F.Cu") (at 203.5 91.5)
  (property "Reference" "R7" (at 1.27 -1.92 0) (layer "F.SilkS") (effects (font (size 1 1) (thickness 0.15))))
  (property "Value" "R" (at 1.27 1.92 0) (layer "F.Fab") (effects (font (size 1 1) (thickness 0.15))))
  (fp_line (start 0.92 0) (end 1.54 0) (stroke (width 0.12) (type solid)) (layer "F.SilkS"))
  (fp_circle (center 0 0) (end 0.92 0) (stroke (width 0.12) (type solid)) (fill none) (layer "F.SilkS"))
  (pad "1" thru_hole circle (at 0 0) (size 1.4 1.4) (drill 0.7) (layers "*.Cu" "*.Mask") (remove_unused_layers no) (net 4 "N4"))
  (pad "2" thru_hole oval (at 2.54 0) (size 1.4 1.4) (drill 0.7) (layers "*.Cu" "*.Mask") (remove_unused_layers no) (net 7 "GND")))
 (gr_rect (start 52 16.5) (end 275 147) (stroke (width 0.05) (type default)) (fill none) (layer "Edge.Cuts"))
 (segment (start 152.4975 109.9975) (end 157.5 115) (width 0.2) (layer "F.Cu") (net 7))
 (segment (start 148 103.995) (end 141.9975 109.9975) (width 0.2) (layer "F.Cu") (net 7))
 (segment (start 141.9975 109.9975) (end 152.4975 109.9975) (width 0.2) (layer "F.Cu") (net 7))
 (segment (start 148 98) (end 148 103.995) (width 0.2) (layer "F.Cu") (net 7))
 (segment (start 141.9975 109.9975) (end 140.995 111) (width 0.2) (layer "F.Cu") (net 7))
 (segment (start 182.54 115) (end 206.04 91.5) (width 0.2) (layer "B.Cu") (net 7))
 (segment (start 157.5 115) (end 182.54 115) (width 0.2) (layer "B.Cu") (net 7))
 (segment (start 227 50.28) (end 225.9 49.18) (width 0.2) (layer "F.Cu") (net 4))
 (segment (start 197.46 46.64) (end 227.455635 46.64) (width 0.2) (layer "B.Cu") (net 2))
 (segment (start 228.1 54.26) (end 227 55.36) (width 0.2) (layer "B.Cu") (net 2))
 (segment (start 227.455635 46.64) (end 228.1 47.284365) (width 0.2) (layer "B.Cu") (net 2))
 (segment (start 146.1 98) (end 197.46 46.64) (width 0.2) (layer "B.Cu") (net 2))
 (segment (start 146.1 120.6) (end 155 129.5) (width 0.2) (layer "B.Cu") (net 2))
 (segment (start 228.1 47.284365) (end 228.1 54.26) (width 0.2) (layer "B.Cu") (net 2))
 (segment (start 146.1 98) (end 146.1 120.6) (width 0.2) (layer "B.Cu") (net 2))
 (segment (start 146.944365 130.6) (end 146.3 129.955635) (width 0.2) (layer "F.Cu") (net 8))
 (segment (start 146.3 129.044365) (end 210.344365 65) (width 0.2) (layer "F.Cu") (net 8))
 (segment (start 175.2 130.6) (end 146.944365 130.6) (width 0.2) (layer "F.Cu") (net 8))
 (segment (start 210.344365 65) (end 216.715635 65) (width 0.2) (layer "F.Cu") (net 8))
 (segment (start 139.095 122.750635) (end 139.095 111) (width 0.2) (layer "F.Cu") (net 8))
 (segment (start 225.9 55.815635) (end 225.9 53.92) (width 0.2) (layer "F.Cu") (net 8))
 (segment (start 181.8 124) (end 175.2 130.6) (width 0.2) (layer "F.Cu") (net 8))
 (segment (start 146.944365 130.6) (end 139.095 122.750635) (width 0.2) (layer "F.Cu") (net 8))
 (segment (start 216.715635 65) (end 225.9 55.815635) (width 0.2) (layer "F.Cu") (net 8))
 (segment (start 146.3 129.955635) (end 146.3 129.044365) (width 0.2) (layer "F.Cu") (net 8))
 (segment (start 208.8 122.5) (end 202.3 116) (width 0.2) (layer "B.Cu") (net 3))
 (segment (start 156.6 116) (end 155.6 115) (width 0.2) (layer "B.Cu") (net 3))
 (segment (start 202.3 116) (end 156.6 116) (width 0.2) (layer "B.Cu") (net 3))
 (segment (start 225.9 105.4) (end 225.9 48.84) (width 0.2) (layer "B.Cu") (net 3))
 (segment (start 208.8 122.5) (end 225.9 105.4) (width 0.2) (layer "B.Cu") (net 3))
 (segment (start 225.9 48.84) (end 227 47.74) (width 0.2) (layer "B.Cu") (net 3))
 (segment (start 103.55 124.625) (end 103.55 112.95) (width 0.2) (layer "F.Cu") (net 5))
 (segment (start 127.5 89) (end 127.5 87.85) (width 0.2) (layer "F.Cu") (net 5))
 (segment (start 103.55 112.95) (end 127.5 89) (width 0.2) (layer "F.Cu") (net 5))
 (segment (start 89.55 82.833452) (end 126.883452 45.5) (width 0.2) (layer "F.Cu") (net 10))
 (segment (start 92.85 90.15) (end 128.15 54.85) (width 0.2) (layer "F.Cu") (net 10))
 (segment (start 128.5 45.5) (end 128.5 43.95) (width 0.2) (layer "F.Cu") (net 10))
 (segment (start 92.85 124.625) (end 92.85 90.15) (width 0.2) (layer "F.Cu") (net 10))
 (segment (start 126.883452 45.5) (end 128.5 45.5) (width 0.2) (layer "F.Cu") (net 10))
 (segment (start 89.55 124.625) (end 89.55 82.833452) (width 0.2) (layer "F.Cu") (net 10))
 (segment (start 201.2 122.5) (end 202.999999 120.700001) (width 0.2) (layer "F.Cu") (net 1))
 (segment (start 147.4 129.5) (end 152.9 124) (width 0.2) (layer "F.Cu") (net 1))
 (segment (start 152.9 124) (end 174.2 124) (width 0.2) (layer "F.Cu") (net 1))
 (segment (start 174.2 124) (end 175.7 122.5) (width 0.2) (layer "F.Cu") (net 1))
 (segment (start 225 121.5) (end 228.1 118.4) (width 0.2) (layer "F.Cu") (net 1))
 (segment (start 228.1 36.14) (end 227 35.04) (width 0.2) (layer "F.Cu") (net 1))
 (segment (start 228.1 118.4) (end 228.1 36.14) (width 0.2) (layer "F.Cu") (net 1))
 (segment (start 224.200001 120.700001) (end 225 121.5) (width 0.2) (layer "F.Cu") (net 1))
 (segment (start 175.7 122.5) (end 201.2 122.5) (width 0.2) (layer "F.Cu") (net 1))
 (segment (start 202.999999 120.700001) (end 224.200001 120.700001) (width 0.2) (layer "F.Cu") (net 1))
 (segment (start 106.85 124.625) (end 106.85 119.55) (width 0.2) (layer "F.Cu") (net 6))
 (segment (start 106.85 119.55) (end 127.65 98.75) (width 0.2) (layer "F.Cu") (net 6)))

